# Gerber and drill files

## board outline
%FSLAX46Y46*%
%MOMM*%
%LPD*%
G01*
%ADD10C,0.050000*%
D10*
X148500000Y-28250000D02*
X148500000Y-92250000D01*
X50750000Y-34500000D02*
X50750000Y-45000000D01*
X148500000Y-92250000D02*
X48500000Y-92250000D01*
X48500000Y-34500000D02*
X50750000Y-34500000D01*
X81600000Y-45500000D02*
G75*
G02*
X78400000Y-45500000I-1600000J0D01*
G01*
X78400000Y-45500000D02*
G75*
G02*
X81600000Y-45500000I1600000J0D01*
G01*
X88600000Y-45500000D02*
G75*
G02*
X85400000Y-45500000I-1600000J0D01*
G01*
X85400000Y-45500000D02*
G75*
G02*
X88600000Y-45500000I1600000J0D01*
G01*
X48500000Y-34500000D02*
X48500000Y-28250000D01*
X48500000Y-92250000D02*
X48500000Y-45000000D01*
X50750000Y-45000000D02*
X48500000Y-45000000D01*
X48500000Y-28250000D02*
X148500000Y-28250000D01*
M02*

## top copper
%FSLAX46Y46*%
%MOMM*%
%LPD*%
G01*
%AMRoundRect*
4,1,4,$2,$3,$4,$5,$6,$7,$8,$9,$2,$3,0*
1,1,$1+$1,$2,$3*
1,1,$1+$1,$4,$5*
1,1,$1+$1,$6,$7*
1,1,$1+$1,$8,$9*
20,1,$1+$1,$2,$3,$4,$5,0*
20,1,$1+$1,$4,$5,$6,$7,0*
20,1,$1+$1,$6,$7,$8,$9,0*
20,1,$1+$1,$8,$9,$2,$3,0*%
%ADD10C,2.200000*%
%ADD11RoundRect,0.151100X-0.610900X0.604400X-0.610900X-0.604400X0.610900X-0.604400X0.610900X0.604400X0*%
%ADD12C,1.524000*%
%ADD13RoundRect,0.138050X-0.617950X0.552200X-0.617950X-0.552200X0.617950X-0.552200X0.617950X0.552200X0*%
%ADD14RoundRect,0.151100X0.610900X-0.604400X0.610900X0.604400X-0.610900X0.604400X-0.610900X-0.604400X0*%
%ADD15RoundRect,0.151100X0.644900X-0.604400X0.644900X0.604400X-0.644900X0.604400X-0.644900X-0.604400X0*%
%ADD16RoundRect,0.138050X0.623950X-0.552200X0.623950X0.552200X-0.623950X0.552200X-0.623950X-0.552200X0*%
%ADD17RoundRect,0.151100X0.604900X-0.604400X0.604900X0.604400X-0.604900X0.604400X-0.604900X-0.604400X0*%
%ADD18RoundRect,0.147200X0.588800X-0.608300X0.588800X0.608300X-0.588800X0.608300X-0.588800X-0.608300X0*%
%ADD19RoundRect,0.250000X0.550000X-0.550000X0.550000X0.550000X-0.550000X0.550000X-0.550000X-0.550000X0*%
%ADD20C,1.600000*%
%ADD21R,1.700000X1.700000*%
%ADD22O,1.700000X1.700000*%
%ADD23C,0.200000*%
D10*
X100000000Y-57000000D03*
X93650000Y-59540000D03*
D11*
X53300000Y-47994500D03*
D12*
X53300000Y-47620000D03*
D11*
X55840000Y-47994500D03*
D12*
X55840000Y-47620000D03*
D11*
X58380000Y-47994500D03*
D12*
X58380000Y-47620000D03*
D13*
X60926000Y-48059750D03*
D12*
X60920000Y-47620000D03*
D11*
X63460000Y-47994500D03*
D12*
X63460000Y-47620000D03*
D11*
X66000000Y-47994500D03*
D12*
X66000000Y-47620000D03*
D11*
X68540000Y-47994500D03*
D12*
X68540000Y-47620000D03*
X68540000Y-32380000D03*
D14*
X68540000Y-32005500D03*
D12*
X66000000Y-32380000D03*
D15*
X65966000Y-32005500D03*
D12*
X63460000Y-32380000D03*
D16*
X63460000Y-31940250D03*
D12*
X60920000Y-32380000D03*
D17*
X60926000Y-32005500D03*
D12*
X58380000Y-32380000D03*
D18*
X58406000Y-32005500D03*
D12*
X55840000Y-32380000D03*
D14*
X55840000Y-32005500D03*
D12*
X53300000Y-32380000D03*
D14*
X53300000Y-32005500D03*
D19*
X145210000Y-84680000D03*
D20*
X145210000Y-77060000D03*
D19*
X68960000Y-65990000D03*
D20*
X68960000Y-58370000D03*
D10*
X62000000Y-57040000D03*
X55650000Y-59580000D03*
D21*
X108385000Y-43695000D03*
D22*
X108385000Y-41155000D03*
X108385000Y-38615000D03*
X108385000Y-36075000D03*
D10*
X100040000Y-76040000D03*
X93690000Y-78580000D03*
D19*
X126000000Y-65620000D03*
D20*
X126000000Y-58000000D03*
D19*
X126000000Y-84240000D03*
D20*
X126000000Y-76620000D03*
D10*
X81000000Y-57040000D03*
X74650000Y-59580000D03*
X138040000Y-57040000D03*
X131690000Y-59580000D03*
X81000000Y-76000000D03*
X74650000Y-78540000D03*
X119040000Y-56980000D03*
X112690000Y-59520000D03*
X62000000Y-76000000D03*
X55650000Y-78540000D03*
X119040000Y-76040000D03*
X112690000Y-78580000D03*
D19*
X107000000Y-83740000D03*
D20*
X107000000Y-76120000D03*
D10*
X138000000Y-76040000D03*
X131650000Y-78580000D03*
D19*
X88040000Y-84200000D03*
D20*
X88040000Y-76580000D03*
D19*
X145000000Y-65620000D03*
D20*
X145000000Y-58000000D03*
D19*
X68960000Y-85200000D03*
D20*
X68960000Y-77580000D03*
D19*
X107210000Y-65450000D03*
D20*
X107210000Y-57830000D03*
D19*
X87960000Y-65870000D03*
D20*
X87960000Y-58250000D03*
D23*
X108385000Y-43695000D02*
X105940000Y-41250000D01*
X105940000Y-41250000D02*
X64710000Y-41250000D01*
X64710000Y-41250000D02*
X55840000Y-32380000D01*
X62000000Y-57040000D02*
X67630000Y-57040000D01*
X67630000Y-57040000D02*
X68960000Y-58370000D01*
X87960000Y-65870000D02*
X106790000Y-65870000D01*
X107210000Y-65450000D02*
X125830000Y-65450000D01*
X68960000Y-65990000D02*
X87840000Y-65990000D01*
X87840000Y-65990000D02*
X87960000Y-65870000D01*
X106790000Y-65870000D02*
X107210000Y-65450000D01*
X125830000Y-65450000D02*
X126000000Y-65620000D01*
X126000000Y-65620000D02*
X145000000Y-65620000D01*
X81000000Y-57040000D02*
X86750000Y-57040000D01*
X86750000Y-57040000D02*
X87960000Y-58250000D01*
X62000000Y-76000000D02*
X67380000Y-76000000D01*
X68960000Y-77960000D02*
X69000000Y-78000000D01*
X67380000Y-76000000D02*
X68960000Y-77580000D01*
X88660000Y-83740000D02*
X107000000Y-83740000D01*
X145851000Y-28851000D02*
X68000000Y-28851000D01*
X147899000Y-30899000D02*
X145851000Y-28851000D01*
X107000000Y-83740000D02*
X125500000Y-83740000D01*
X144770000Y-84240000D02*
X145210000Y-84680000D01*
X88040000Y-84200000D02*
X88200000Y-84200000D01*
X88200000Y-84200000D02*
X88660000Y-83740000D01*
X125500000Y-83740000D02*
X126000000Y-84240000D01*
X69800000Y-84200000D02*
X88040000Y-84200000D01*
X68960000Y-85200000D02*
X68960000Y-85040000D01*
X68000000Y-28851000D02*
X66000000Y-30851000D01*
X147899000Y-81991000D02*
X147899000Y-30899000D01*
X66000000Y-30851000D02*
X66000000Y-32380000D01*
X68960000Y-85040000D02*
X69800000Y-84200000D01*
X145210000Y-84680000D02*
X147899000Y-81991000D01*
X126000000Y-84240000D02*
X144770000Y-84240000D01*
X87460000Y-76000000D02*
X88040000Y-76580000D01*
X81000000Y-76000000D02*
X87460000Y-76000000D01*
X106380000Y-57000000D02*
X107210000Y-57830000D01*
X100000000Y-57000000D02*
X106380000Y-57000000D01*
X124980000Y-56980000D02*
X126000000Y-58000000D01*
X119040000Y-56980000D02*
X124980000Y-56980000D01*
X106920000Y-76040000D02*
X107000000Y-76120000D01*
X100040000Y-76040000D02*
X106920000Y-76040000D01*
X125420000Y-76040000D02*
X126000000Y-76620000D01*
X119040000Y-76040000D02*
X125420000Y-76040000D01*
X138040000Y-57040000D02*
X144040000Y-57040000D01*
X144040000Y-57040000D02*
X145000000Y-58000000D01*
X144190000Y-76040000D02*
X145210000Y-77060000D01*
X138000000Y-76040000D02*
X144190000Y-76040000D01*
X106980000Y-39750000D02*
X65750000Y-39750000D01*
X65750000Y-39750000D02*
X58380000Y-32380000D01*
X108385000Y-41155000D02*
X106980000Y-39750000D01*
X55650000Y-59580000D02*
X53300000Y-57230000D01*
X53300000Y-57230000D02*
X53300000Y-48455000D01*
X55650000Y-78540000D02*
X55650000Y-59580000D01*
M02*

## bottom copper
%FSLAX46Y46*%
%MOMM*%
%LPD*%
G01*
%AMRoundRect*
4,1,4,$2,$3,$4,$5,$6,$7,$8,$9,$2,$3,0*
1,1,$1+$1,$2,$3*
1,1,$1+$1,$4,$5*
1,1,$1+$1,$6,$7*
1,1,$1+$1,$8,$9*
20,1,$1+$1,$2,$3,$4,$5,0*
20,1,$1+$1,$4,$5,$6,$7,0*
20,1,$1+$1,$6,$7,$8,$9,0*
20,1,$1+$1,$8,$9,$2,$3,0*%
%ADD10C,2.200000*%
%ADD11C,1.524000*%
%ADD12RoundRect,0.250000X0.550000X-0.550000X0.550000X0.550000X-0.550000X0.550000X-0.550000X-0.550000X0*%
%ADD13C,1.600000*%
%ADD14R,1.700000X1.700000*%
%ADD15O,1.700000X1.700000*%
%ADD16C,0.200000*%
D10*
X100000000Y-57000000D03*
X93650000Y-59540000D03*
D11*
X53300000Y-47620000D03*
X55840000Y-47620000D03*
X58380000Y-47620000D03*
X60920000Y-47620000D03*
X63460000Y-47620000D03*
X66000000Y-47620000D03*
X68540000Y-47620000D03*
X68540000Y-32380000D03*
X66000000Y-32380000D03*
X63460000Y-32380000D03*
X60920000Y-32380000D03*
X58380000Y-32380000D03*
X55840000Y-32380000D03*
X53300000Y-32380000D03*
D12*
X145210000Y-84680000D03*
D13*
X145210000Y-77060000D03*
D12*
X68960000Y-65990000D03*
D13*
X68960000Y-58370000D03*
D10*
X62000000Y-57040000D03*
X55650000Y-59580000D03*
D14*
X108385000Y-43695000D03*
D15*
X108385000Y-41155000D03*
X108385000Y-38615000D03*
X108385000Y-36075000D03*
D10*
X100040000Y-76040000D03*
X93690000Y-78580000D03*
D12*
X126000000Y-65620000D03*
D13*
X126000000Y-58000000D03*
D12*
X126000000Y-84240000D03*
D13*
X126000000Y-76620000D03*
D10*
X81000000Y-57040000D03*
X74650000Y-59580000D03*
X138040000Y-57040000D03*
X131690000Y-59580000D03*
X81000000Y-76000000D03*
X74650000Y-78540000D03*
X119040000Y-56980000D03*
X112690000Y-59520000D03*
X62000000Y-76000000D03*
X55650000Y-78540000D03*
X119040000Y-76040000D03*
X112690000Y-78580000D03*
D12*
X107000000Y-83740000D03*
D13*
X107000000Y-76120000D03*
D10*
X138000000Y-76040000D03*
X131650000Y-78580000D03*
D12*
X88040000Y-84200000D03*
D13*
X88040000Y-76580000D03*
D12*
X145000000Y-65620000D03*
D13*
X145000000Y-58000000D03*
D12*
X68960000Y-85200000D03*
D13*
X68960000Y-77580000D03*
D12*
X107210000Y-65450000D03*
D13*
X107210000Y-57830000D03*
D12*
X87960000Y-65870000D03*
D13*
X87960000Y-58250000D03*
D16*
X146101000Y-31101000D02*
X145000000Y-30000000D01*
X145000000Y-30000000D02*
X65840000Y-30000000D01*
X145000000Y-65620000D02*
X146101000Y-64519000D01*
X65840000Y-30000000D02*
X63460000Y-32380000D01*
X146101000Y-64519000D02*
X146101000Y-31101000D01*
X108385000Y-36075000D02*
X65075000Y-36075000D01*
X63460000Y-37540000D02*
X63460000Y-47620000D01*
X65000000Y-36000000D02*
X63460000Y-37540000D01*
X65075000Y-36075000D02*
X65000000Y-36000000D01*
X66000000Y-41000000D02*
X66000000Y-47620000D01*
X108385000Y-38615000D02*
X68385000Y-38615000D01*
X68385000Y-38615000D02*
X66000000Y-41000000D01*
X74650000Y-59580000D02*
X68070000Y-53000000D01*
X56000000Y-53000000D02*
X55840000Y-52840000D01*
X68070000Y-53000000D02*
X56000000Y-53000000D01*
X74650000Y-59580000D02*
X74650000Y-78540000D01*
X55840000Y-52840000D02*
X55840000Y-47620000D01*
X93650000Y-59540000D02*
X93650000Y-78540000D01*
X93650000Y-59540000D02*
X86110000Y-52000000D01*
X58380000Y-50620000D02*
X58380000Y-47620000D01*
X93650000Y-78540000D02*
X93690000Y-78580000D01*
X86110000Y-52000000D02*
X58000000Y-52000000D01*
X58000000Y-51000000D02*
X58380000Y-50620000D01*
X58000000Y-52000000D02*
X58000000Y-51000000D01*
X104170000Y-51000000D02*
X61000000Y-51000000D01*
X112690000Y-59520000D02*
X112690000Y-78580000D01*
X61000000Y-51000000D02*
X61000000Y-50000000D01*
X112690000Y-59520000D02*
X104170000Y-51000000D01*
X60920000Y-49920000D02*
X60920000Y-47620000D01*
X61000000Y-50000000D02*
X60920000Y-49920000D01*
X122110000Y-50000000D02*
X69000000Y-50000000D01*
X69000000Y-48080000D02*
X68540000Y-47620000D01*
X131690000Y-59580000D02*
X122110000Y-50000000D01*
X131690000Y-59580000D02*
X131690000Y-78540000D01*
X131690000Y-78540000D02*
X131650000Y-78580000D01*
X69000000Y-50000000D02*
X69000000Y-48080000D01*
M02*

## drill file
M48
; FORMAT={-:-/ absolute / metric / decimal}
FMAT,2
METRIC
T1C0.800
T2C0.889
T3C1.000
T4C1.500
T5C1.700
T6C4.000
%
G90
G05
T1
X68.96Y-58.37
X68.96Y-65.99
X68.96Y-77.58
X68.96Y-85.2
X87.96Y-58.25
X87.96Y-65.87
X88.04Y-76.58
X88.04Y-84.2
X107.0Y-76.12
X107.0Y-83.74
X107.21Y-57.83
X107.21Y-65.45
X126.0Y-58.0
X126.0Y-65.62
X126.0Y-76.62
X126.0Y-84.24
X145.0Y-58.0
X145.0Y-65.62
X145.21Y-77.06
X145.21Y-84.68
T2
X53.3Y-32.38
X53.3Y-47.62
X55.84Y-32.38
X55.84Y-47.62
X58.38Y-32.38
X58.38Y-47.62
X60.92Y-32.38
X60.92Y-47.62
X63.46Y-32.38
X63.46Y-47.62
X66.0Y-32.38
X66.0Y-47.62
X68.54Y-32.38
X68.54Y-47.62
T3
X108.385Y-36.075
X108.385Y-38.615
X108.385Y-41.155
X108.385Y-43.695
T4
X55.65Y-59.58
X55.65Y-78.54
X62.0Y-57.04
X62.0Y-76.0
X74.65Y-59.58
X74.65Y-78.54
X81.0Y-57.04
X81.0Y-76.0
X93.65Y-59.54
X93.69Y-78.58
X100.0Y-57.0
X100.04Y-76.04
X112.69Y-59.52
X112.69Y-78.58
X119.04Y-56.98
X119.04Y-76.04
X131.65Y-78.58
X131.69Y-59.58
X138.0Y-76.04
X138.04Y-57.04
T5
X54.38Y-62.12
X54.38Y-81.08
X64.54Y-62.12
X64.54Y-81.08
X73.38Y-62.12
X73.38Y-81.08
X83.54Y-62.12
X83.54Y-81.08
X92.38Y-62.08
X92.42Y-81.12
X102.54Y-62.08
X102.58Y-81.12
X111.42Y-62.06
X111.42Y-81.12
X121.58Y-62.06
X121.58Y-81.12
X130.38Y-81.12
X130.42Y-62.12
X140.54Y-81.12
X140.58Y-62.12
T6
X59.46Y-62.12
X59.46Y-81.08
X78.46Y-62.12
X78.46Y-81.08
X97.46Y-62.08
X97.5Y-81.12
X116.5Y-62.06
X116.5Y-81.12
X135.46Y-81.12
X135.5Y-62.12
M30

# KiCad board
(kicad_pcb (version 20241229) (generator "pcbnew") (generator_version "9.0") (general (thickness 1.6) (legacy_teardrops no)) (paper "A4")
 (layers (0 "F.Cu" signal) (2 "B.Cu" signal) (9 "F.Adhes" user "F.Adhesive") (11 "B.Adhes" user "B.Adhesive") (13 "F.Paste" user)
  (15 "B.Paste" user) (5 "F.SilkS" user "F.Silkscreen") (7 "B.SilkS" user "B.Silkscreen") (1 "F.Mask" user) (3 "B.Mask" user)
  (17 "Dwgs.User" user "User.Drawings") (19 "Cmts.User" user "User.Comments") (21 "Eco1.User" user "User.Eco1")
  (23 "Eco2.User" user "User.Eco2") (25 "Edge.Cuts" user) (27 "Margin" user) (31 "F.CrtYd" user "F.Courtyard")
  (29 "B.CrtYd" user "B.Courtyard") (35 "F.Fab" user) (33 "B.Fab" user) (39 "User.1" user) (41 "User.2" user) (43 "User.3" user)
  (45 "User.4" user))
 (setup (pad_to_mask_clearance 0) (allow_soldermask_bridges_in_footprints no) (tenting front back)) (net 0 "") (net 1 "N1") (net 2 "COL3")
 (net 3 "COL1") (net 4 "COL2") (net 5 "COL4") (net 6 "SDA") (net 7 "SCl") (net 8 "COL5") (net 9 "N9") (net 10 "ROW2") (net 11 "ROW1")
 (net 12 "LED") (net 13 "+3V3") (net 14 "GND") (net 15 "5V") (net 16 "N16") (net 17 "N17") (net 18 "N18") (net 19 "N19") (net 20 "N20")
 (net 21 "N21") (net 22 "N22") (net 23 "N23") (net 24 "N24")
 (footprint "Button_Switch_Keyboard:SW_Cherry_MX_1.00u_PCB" (layer "F.Cu") (at 100 57)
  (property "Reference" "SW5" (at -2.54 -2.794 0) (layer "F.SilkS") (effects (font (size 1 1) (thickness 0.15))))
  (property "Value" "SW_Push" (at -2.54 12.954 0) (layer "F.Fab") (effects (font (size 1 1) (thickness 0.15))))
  (pad "" np_thru_hole circle (at -7.62 5.08) (size 1.7 1.7) (drill 1.7) (layers "*.Cu" "*.Mask"))
  (pad "" np_thru_hole circle (at -2.54 5.08) (size 4 4) (drill 4) (layers "*.Cu" "*.Mask"))
  (pad "" np_thru_hole circle (at 2.54 5.08) (size 1.7 1.7) (drill 1.7) (layers "*.Cu" "*.Mask"))
  (pad "1" thru_hole circle (at 0 0) (size 2.2 2.2) (drill 1.5) (layers "*.Cu" "*.Mask") (remove_unused_layers no) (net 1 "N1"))
  (pad "2" thru_hole circle (at -6.35 2.54) (size 2.2 2.2) (drill 1.5) (layers "*.Cu" "*.Mask") (remove_unused_layers no) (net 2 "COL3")))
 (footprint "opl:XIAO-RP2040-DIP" (layer "F.Cu") (at 60.92 40 90)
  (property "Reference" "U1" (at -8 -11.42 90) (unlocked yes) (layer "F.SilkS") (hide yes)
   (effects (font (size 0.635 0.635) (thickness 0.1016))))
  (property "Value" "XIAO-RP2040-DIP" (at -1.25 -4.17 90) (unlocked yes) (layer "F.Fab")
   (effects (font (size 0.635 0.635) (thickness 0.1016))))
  (pad "1" smd roundrect (at -7.9945 -7.62 270) (size 1.511 1.524) (layers "F.Cu" "F.Mask") (roundrect_rratio 0.1) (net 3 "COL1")
   (thermal_bridge_angle 45))
  (pad "1" thru_hole circle (at -7.62 -7.62 270) (size 1.524 1.524) (drill 0.889) (layers "*.Cu" "*.Mask") (remove_unused_layers no)
   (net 3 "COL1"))
  (pad "2" smd roundrect (at -7.9945 -5.08 270) (size 1.511 1.524) (layers "F.Cu" "F.Mask") (roundrect_rratio 0.1) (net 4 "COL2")
   (thermal_bridge_angle 45))
  (pad "2" thru_hole circle (at -7.62 -5.08 270) (size 1.524 1.524) (drill 0.889) (layers "*.Cu" "*.Mask") (remove_unused_layers no)
   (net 4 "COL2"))
  (pad "3" smd roundrect (at -7.9945 -2.54 270) (size 1.511 1.524) (layers "F.Cu" "F.Mask") (roundrect_rratio 0.1) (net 2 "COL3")
   (thermal_bridge_angle 45))
  (pad "3" thru_hole circle (at -7.62 -2.54 270) (size 1.524 1.524) (drill 0.889) (layers "*.Cu" "*.Mask") (remove_unused_layers no)
   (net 2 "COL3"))
  (pad "4" smd roundrect (at -8.05975 0.006 270) (size 1.3805 1.512) (layers "F.Cu" "F.Mask") (roundrect_rratio 0.1) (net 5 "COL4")
   (thermal_bridge_angle 45))
  (pad "4" thru_hole circle (at -7.62 0 270) (size 1.524 1.524) (drill 0.889) (layers "*.Cu" "*.Mask") (remove_unused_layers no)
   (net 5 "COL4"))
  (pad "5" smd roundrect (at -7.9945 2.54 270) (size 1.511 1.524) (layers "F.Cu" "F.Mask") (roundrect_rratio 0.1) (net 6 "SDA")
   (thermal_bridge_angle 45))
  (pad "5" thru_hole circle (at -7.62 2.54 270) (size 1.524 1.524) (drill 0.889) (layers "*.Cu" "*.Mask") (remove_unused_layers no)
   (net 6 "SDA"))
  (pad "6" smd roundrect (at -7.9945 5.08 270) (size 1.511 1.524) (layers "F.Cu" "F.Mask") (roundrect_rratio 0.1) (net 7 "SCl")
   (thermal_bridge_angle 45))
  (pad "6" thru_hole circle (at -7.62 5.08 270) (size 1.524 1.524) (drill 0.889) (layers "*.Cu" "*.Mask") (remove_unused_layers no)
   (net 7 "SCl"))
  (pad "7" smd roundrect (at -7.9945 7.62 270) (size 1.511 1.524) (layers "F.Cu" "F.Mask") (roundrect_rratio 0.1) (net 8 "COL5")
   (thermal_bridge_angle 45))
  (pad "7" thru_hole circle (at -7.62 7.62 270) (size 1.524 1.524) (drill 0.889) (layers "*.Cu" "*.Mask") (remove_unused_layers no)
   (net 8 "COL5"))
  (pad "8" thru_hole circle (at 7.62 7.62 90) (size 1.524 1.524) (drill 0.889) (layers "*.Cu" "*.Mask") (remove_unused_layers no)
   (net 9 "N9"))
  (pad "8" smd roundrect (at 7.9945 7.62 90) (size 1.511 1.524) (layers "F.Cu" "F.Mask") (roundrect_rratio 0.1) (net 9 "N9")
   (thermal_bridge_angle 45))
  (pad "9" thru_hole circle (at 7.62 5.08 90) (size 1.524 1.524) (drill 0.889) (layers "*.Cu" "*.Mask") (remove_unused_layers no)
   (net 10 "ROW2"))
  (pad "9" smd roundrect (at 7.9945 5.046 90) (size 1.511 1.592) (layers "F.Cu" "F.Mask") (roundrect_rratio 0.1) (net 10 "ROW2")
   (thermal_bridge_angle 45))
  (pad "10" thru_hole circle (at 7.62 2.54 90) (size 1.524 1.524) (drill 0.889) (layers "*.Cu" "*.Mask") (remove_unused_layers no)
   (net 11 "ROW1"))
  (pad "10" smd roundrect (at 8.05975 2.54 90) (size 1.3805 1.524) (layers "F.Cu" "F.Mask") (roundrect_rratio 0.1) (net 11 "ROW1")
   (thermal_bridge_angle 45))
  (pad "11" thru_hole circle (at 7.62 0 90) (size 1.524 1.524) (drill 0.889) (layers "*.Cu" "*.Mask") (remove_unused_layers no)
   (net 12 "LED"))
  (pad "11" smd roundrect (at 7.9945 0.006 90) (size 1.511 1.512) (layers "F.Cu" "F.Mask") (roundrect_rratio 0.1) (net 12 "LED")
   (thermal_bridge_angle 45))
  (pad "12" thru_hole circle (at 7.62 -2.54 90) (size 1.524 1.524) (drill 0.889) (layers "*.Cu" "*.Mask") (remove_unused_layers no)
   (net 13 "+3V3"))
  (pad "12" smd roundrect (at 7.9945 -2.514 90) (size 1.511 1.472) (layers "F.Cu" "F.Mask") (roundrect_rratio 0.1) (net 13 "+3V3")
   (thermal_bridge_angle 45))
  (pad "13" thru_hole circle (at 7.62 -5.08 90) (size 1.524 1.524) (drill 0.889) (layers "*.Cu" "*.Mask") (remove_unused_layers no)
   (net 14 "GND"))
  (pad "13" smd roundrect (at 7.9945 -5.08 90) (size 1.511 1.524) (layers "F.Cu" "F.Mask") (roundrect_rratio 0.1) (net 14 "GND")
   (thermal_bridge_angle 45))
  (pad "14" thru_hole circle (at 7.62 -7.62 90) (size 1.524 1.524) (drill 0.889) (layers "*.Cu" "*.Mask") (remove_unused_layers no)
   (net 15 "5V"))
  (pad "14" smd roundrect (at 7.9945 -7.62 90) (size 1.511 1.524) (layers "F.Cu" "F.Mask") (roundrect_rratio 0.1) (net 15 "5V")
   (thermal_bridge_angle 45)))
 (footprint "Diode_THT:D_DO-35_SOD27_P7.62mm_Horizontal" (layer "F.Cu") (at 145.21 84.68 90)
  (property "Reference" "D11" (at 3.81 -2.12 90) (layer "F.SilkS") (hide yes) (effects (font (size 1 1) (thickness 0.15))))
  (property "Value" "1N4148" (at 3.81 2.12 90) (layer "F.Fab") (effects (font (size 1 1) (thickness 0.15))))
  (pad "1" thru_hole roundrect (at 0 0 90) (size 1.6 1.6) (drill 0.8) (layers "*.Cu" "*.Mask") (remove_unused_layers no)
   (roundrect_rratio 0.15625) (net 10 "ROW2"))
  (pad "2" thru_hole circle (at 7.62 0 90) (size 1.6 1.6) (drill 0.8) (layers "*.Cu" "*.Mask") (remove_unused_layers no) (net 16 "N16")))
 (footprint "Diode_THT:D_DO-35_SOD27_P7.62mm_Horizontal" (layer "F.Cu") (at 68.96 65.99 90)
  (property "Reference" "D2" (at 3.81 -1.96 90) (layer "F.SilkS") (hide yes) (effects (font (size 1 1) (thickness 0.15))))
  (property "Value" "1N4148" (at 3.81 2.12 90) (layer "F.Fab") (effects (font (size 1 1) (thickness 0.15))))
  (pad "1" thru_hole roundrect (at 0 0 90) (size 1.6 1.6) (drill 0.8) (layers "*.Cu" "*.Mask") (remove_unused_layers no)
   (roundrect_rratio 0.15625) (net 11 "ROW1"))
  (pad "2" thru_hole circle (at 7.62 0 90) (size 1.6 1.6) (drill 0.8) (layers "*.Cu" "*.Mask") (remove_unused_layers no) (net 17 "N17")))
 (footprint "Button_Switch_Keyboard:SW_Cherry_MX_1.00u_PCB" (layer "F.Cu") (at 62 57.04)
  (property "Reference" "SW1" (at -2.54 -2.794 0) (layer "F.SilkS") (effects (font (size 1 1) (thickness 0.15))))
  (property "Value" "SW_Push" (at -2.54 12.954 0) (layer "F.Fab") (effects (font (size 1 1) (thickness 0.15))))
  (pad "" np_thru_hole circle (at -7.62 5.08) (size 1.7 1.7) (drill 1.7) (layers "*.Cu" "*.Mask"))
  (pad "" np_thru_hole circle (at -2.54 5.08) (size 4 4) (drill 4) (layers "*.Cu" "*.Mask"))
  (pad "" np_thru_hole circle (at 2.54 5.08) (size 1.7 1.7) (drill 1.7) (layers "*.Cu" "*.Mask"))
  (pad "1" thru_hole circle (at 0 0) (size 2.2 2.2) (drill 1.5) (layers "*.Cu" "*.Mask") (remove_unused_layers no) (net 17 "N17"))
  (pad "2" thru_hole circle (at -6.35 2.54) (size 2.2 2.2) (drill 1.5) (layers "*.Cu" "*.Mask") (remove_unused_layers no) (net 3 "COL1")))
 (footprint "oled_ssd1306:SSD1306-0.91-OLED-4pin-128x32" (layer "F.Cu") (at 144.885 45.885 180)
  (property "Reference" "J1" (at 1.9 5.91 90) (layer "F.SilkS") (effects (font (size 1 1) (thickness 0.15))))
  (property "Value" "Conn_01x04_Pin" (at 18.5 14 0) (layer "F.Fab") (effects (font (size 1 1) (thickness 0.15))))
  (pad "1" thru_hole rect (at 36.5 2.19 180) (size 1.7 1.7) (drill 1) (layers "*.Cu" "*.Mask") (remove_unused_layers no) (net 14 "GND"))
  (pad "2" thru_hole oval (at 36.5 4.73 180) (size 1.7 1.7) (drill 1) (layers "*.Cu" "*.Mask") (remove_unused_layers no) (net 13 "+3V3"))
  (pad "3" thru_hole oval (at 36.5 7.27 180) (size 1.7 1.7) (drill 1) (layers "*.Cu" "*.Mask") (remove_unused_layers no) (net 7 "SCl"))
  (pad "4" thru_hole oval (at 36.5 9.81 180) (size 1.7 1.7) (drill 1) (layers "*.Cu" "*.Mask") (remove_unused_layers no) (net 6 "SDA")))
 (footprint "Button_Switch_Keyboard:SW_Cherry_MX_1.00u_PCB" (layer "F.Cu") (at 100.04 76.04)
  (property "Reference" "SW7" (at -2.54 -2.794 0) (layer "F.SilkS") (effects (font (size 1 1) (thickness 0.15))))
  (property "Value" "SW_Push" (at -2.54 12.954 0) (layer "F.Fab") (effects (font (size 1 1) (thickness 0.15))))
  (pad "" np_thru_hole circle (at -7.62 5.08) (size 1.7 1.7) (drill 1.7) (layers "*.Cu" "*.Mask"))
  (pad "" np_thru_hole circle (at -2.54 5.08) (size 4 4) (drill 4) (layers "*.Cu" "*.Mask"))
  (pad "" np_thru_hole circle (at 2.54 5.08) (size 1.7 1.7) (drill 1.7) (layers "*.Cu" "*.Mask"))
  (pad "1" thru_hole circle (at 0 0) (size 2.2 2.2) (drill 1.5) (layers "*.Cu" "*.Mask") (remove_unused_layers no) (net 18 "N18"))
  (pad "2" thru_hole circle (at -6.35 2.54) (size 2.2 2.2) (drill 1.5) (layers "*.Cu" "*.Mask") (remove_unused_layers no) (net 2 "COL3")))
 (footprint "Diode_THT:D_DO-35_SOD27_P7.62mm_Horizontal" (layer "F.Cu") (at 126 65.62 90)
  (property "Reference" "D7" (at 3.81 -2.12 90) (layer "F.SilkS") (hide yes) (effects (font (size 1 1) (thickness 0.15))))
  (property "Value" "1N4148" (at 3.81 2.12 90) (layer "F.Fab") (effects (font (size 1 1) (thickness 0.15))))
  (pad "1" thru_hole roundrect (at 0 0 90) (size 1.6 1.6) (drill 0.8) (layers "*.Cu" "*.Mask") (remove_unused_layers no)
   (roundrect_rratio 0.15625) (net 11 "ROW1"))
  (pad "2" thru_hole circle (at 7.62 0 90) (size 1.6 1.6) (drill 0.8) (layers "*.Cu" "*.Mask") (remove_unused_layers no) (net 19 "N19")))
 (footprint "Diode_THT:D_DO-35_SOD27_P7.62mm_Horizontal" (layer "F.Cu") (at 126 84.24 90)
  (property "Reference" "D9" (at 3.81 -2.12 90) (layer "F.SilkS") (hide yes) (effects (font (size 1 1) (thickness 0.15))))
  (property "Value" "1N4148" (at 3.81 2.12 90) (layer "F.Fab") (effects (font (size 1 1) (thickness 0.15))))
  (pad "1" thru_hole roundrect (at 0 0 90) (size 1.6 1.6) (drill 0.8) (layers "*.Cu" "*.Mask") (remove_unused_layers no)
   (roundrect_rratio 0.15625) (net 10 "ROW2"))
  (pad "2" thru_hole circle (at 7.62 0 90) (size 1.6 1.6) (drill 0.8) (layers "*.Cu" "*.Mask") (remove_unused_layers no) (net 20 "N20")))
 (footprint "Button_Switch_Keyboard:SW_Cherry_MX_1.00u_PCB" (layer "F.Cu") (at 81 57.04)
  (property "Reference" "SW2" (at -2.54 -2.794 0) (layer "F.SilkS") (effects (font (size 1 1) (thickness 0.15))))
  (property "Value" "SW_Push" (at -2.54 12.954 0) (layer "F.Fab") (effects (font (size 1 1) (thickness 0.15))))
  (pad "" np_thru_hole circle (at -7.62 5.08) (size 1.7 1.7) (drill 1.7) (layers "*.Cu" "*.Mask"))
  (pad "" np_thru_hole circle (at -2.54 5.08) (size 4 4) (drill 4) (layers "*.Cu" "*.Mask"))
  (pad "" np_thru_hole circle (at 2.54 5.08) (size 1.7 1.7) (drill 1.7) (layers "*.Cu" "*.Mask"))
  (pad "1" thru_hole circle (at 0 0) (size 2.2 2.2) (drill 1.5) (layers "*.Cu" "*.Mask") (remove_unused_layers no) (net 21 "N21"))
  (pad "2" thru_hole circle (at -6.35 2.54) (size 2.2 2.2) (drill 1.5) (layers "*.Cu" "*.Mask") (remove_unused_layers no) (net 4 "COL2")))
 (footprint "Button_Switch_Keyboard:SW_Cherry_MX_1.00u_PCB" (layer "F.Cu") (at 138.04 57.04)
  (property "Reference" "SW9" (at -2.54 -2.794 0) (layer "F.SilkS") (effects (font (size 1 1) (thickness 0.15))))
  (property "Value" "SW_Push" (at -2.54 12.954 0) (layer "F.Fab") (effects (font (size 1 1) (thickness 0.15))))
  (pad "" np_thru_hole circle (at -7.62 5.08) (size 1.7 1.7) (drill 1.7) (layers "*.Cu" "*.Mask"))
  (pad "" np_thru_hole circle (at -2.54 5.08) (size 4 4) (drill 4) (layers "*.Cu" "*.Mask"))
  (pad "" np_thru_hole circle (at 2.54 5.08) (size 1.7 1.7) (drill 1.7) (layers "*.Cu" "*.Mask"))
  (pad "1" thru_hole circle (at 0 0) (size 2.2 2.2) (drill 1.5) (layers "*.Cu" "*.Mask") (remove_unused_layers no) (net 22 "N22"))
  (pad "2" thru_hole circle (at -6.35 2.54) (size 2.2 2.2) (drill 1.5) (layers "*.Cu" "*.Mask") (remove_unused_layers no) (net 8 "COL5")))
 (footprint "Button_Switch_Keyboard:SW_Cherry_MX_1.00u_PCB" (layer "F.Cu") (at 81 76)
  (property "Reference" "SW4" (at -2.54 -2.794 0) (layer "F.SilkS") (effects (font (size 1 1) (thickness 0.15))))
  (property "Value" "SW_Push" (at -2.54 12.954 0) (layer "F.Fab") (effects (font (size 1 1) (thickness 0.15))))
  (pad "" np_thru_hole circle (at -7.62 5.08) (size 1.7 1.7) (drill 1.7) (layers "*.Cu" "*.Mask"))
  (pad "" np_thru_hole circle (at -2.54 5.08) (size 4 4) (drill 4) (layers "*.Cu" "*.Mask"))
  (pad "" np_thru_hole circle (at 2.54 5.08) (size 1.7 1.7) (drill 1.7) (layers "*.Cu" "*.Mask"))
  (pad "1" thru_hole circle (at 0 0) (size 2.2 2.2) (drill 1.5) (layers "*.Cu" "*.Mask") (remove_unused_layers no) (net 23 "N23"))
  (pad "2" thru_hole circle (at -6.35 2.54) (size 2.2 2.2) (drill 1.5) (layers "*.Cu" "*.Mask") (remove_unused_layers no) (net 4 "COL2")))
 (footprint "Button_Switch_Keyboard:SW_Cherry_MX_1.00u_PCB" (layer "F.Cu") (at 119.04 56.98)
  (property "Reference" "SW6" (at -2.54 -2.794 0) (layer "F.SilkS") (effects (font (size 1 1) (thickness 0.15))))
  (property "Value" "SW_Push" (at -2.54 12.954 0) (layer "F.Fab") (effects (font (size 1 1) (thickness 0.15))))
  (pad "" np_thru_hole circle (at -7.62 5.08) (size 1.7 1.7) (drill 1.7) (layers "*.Cu" "*.Mask"))
  (pad "" np_thru_hole circle (at -2.54 5.08) (size 4 4) (drill 4) (layers "*.Cu" "*.Mask"))
  (pad "" np_thru_hole circle (at 2.54 5.08) (size 1.7 1.7) (drill 1.7) (layers "*.Cu" "*.Mask"))
  (pad "1" thru_hole circle (at 0 0) (size 2.2 2.2) (drill 1.5) (layers "*.Cu" "*.Mask") (remove_unused_layers no) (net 19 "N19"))
  (pad "2" thru_hole circle (at -6.35 2.54) (size 2.2 2.2) (drill 1.5) (layers "*.Cu" "*.Mask") (remove_unused_layers no) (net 5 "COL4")))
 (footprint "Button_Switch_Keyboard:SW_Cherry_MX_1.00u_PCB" (layer "F.Cu") (at 62 76)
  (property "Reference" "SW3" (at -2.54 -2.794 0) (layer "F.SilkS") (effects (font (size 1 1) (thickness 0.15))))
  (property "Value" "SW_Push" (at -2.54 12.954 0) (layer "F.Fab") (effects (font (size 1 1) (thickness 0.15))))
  (pad "" np_thru_hole circle (at -7.62 5.08) (size 1.7 1.7) (drill 1.7) (layers "*.Cu" "*.Mask"))
  (pad "" np_thru_hole circle (at -2.54 5.08) (size 4 4) (drill 4) (layers "*.Cu" "*.Mask"))
  (pad "" np_thru_hole circle (at 2.54 5.08) (size 1.7 1.7) (drill 1.7) (layers "*.Cu" "*.Mask"))
  (pad "1" thru_hole circle (at 0 0) (size 2.2 2.2) (drill 1.5) (layers "*.Cu" "*.Mask") (remove_unused_layers no) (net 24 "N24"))
  (pad "2" thru_hole circle (at -6.35 2.54) (size 2.2 2.2) (drill 1.5) (layers "*.Cu" "*.Mask") (remove_unused_layers no) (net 3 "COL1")))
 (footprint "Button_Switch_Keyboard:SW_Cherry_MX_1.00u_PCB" (layer "F.Cu") (at 119.04 76.04)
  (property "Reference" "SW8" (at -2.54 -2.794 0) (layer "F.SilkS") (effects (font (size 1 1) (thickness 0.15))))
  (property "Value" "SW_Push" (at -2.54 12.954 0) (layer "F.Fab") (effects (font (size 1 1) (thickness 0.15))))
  (pad "" np_thru_hole circle (at -7.62 5.08) (size 1.7 1.7) (drill 1.7) (layers "*.Cu" "*.Mask"))
  (pad "" np_thru_hole circle (at -2.54 5.08) (size 4 4) (drill 4) (layers "*.Cu" "*.Mask"))
  (pad "" np_thru_hole circle (at 2.54 5.08) (size 1.7 1.7) (drill 1.7) (layers "*.Cu" "*.Mask"))
  (pad "1" thru_hole circle (at 0 0) (size 2.2 2.2) (drill 1.5) (layers "*.Cu" "*.Mask") (remove_unused_layers no) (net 20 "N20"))
  (pad "2" thru_hole circle (at -6.35 2.54) (size 2.2 2.2) (drill 1.5) (layers "*.Cu" "*.Mask") (remove_unused_layers no) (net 5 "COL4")))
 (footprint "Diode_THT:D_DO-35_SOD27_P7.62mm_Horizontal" (layer "F.Cu") (at 107 83.74 90)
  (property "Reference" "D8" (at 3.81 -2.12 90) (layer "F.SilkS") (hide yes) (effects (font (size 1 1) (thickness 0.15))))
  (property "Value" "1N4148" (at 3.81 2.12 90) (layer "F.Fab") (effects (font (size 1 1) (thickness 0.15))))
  (pad "1" thru_hole roundrect (at 0 0 90) (size 1.6 1.6) (drill 0.8) (layers "*.Cu" "*.Mask") (remove_unused_layers no)
   (roundrect_rratio 0.15625) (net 10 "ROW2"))
  (pad "2" thru_hole circle (at 7.62 0 90) (size 1.6 1.6) (drill 0.8) (layers "*.Cu" "*.Mask") (remove_unused_layers no) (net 18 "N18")))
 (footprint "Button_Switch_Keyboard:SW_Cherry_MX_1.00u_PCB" (layer "F.Cu") (at 138 76.04)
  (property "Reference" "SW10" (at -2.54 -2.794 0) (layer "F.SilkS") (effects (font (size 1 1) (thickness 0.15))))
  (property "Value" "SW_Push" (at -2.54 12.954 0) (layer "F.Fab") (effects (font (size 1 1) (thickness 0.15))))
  (pad "" np_thru_hole circle (at -7.62 5.08) (size 1.7 1.7) (drill 1.7) (layers "*.Cu" "*.Mask"))
  (pad "" np_thru_hole circle (at -2.54 5.08) (size 4 4) (drill 4) (layers "*.Cu" "*.Mask"))
  (pad "" np_thru_hole circle (at 2.54 5.08) (size 1.7 1.7) (drill 1.7) (layers "*.Cu" "*.Mask"))
  (pad "1" thru_hole circle (at 0 0) (size 2.2 2.2) (drill 1.5) (layers "*.Cu" "*.Mask") (remove_unused_layers no) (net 16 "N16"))
  (pad "2" thru_hole circle (at -6.35 2.54) (size 2.2 2.2) (drill 1.5) (layers "*.Cu" "*.Mask") (remove_unused_layers no) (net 8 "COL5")))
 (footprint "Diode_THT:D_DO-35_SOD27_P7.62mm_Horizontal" (layer "F.Cu") (at 88.04 84.2 90)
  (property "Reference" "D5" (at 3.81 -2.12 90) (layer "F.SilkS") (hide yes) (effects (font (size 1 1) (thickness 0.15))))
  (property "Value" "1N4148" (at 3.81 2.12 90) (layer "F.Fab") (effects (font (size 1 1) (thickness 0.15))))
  (pad "1" thru_hole roundrect (at 0 0 90) (size 1.6 1.6) (drill 0.8) (layers "*.Cu" "*.Mask") (remove_unused_layers no)
   (roundrect_rratio 0.15625) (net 10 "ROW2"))
  (pad "2" thru_hole circle (at 7.62 0 90) (size 1.6 1.6) (drill 0.8) (layers "*.Cu" "*.Mask") (remove_unused_layers no) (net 23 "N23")))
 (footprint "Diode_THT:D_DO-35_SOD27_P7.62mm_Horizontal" (layer "F.Cu") (at 145 65.62 90)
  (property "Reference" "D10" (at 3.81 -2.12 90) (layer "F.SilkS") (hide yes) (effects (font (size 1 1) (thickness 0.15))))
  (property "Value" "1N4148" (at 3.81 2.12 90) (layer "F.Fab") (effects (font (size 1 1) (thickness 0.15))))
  (pad "1" thru_hole roundrect (at 0 0 90) (size 1.6 1.6) (drill 0.8) (layers "*.Cu" "*.Mask") (remove_unused_layers no)
   (roundrect_rratio 0.15625) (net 11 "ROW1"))
  (pad "2" thru_hole circle (at 7.62 0 90) (size 1.6 1.6) (drill 0.8) (layers "*.Cu" "*.Mask") (remove_unused_layers no) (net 22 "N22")))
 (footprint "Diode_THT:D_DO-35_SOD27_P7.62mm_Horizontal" (layer "F.Cu") (at 68.96 85.2 90)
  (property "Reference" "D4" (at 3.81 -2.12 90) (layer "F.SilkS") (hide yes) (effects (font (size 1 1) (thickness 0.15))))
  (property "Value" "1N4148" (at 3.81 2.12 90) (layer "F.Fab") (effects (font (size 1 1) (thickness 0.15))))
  (pad "1" thru_hole roundrect (at 0 0 90) (size 1.6 1.6) (drill 0.8) (layers "*.Cu" "*.Mask") (remove_unused_layers no)
   (roundrect_rratio 0.15625) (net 10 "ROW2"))
  (pad "2" thru_hole circle (at 7.62 0 90) (size 1.6 1.6) (drill 0.8) (layers "*.Cu" "*.Mask") (remove_unused_layers no) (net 24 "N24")))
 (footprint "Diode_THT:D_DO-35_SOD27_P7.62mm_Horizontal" (layer "F.Cu") (at 107.21 65.45 90)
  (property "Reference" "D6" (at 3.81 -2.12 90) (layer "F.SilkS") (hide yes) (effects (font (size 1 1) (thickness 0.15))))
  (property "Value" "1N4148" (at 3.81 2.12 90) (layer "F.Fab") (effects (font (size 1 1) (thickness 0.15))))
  (pad "1" thru_hole roundrect (at 0 0 90) (size 1.6 1.6) (drill 0.8) (layers "*.Cu" "*.Mask") (remove_unused_layers no)
   (roundrect_rratio 0.15625) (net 11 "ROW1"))
  (pad "2" thru_hole circle (at 7.62 0 90) (size 1.6 1.6) (drill 0.8) (layers "*.Cu" "*.Mask") (remove_unused_layers no) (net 1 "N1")))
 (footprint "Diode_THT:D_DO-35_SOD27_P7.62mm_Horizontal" (layer "F.Cu") (at 87.96 65.87 90)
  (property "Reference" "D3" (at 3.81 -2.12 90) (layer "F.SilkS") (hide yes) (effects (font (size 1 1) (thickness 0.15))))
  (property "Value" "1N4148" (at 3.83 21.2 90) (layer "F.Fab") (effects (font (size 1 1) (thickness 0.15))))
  (pad "1" thru_hole roundrect (at 0 0 90) (size 1.6 1.6) (drill 0.8) (layers "*.Cu" "*.Mask") (remove_unused_layers no)
   (roundrect_rratio 0.15625) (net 11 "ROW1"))
  (pad "2" thru_hole circle (at 7.62 0 90) (size 1.6 1.6) (drill 0.8) (layers "*.Cu" "*.Mask") (remove_unused_layers no) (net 21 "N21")))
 (gr_line (start 148.5 28.25) (end 148.5 92.25) (stroke (width 0.05) (type default)) (layer "Edge.Cuts"))
 (gr_line (start 50.75 34.5) (end 50.75 45) (stroke (width 0.05) (type default)) (layer "Edge.Cuts"))
 (gr_line (start 148.5 92.25) (end 48.5 92.25) (stroke (width 0.05) (type default)) (layer "Edge.Cuts"))
 (gr_line (start 48.5 34.5) (end 50.75 34.5) (stroke (width 0.05) (type default)) (layer "Edge.Cuts"))
 (gr_circle (center 80 45.5) (end 81.6 45.5) (stroke (width 0.05) (type solid)) (fill no) (layer "Edge.Cuts"))
 (gr_circle (center 87 45.5) (end 88.6 45.5) (stroke (width 0.05) (type solid)) (fill no) (layer "Edge.Cuts"))
 (gr_line (start 48.5 34.5) (end 48.5 28.25) (stroke (width 0.05) (type default)) (layer "Edge.Cuts"))
 (gr_line (start 48.5 92.25) (end 48.5 45) (stroke (width 0.05) (type default)) (layer "Edge.Cuts"))
 (gr_line (start 50.75 45) (end 48.5 45) (stroke (width 0.05) (type default)) (layer "Edge.Cuts"))
 (gr_line (start 48.5 28.25) (end 148.5 28.25) (stroke (width 0.05) (type default)) (layer "Edge.Cuts"))
 (segment (start 108.385 43.695) (end 105.94 41.25) (width 0.2) (layer "F.Cu") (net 14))
 (segment (start 105.94 41.25) (end 64.71 41.25) (width 0.2) (layer "F.Cu") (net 14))
 (segment (start 64.71 41.25) (end 55.84 32.38) (width 0.2) (layer "F.Cu") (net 14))
 (segment (start 62 57.04) (end 67.63 57.04) (width 0.2) (layer "F.Cu") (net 17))
 (segment (start 67.63 57.04) (end 68.96 58.37) (width 0.2) (layer "F.Cu") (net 17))
 (segment (start 87.96 65.87) (end 106.79 65.87) (width 0.2) (layer "F.Cu") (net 11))
 (segment (start 107.21 65.45) (end 125.83 65.45) (width 0.2) (layer "F.Cu") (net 11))
 (segment (start 68.96 65.99) (end 87.84 65.99) (width 0.2) (layer "F.Cu") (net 11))
 (segment (start 87.84 65.99) (end 87.96 65.87) (width 0.2) (layer "F.Cu") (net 11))
 (segment (start 106.79 65.87) (end 107.21 65.45) (width 0.2) (layer "F.Cu") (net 11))
 (segment (start 125.83 65.45) (end 126 65.62) (width 0.2) (layer "F.Cu") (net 11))
 (segment (start 126 65.62) (end 145 65.62) (width 0.2) (layer "F.Cu") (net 11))
 (segment (start 146.101 31.101) (end 145 30) (width 0.2) (layer "B.Cu") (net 11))
 (segment (start 145 30) (end 65.84 30) (width 0.2) (layer "B.Cu") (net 11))
 (segment (start 145 65.62) (end 146.101 64.519) (width 0.2) (layer "B.Cu") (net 11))
 (segment (start 65.84 30) (end 63.46 32.38) (width 0.2) (layer "B.Cu") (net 11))
 (segment (start 146.101 64.519) (end 146.101 31.101) (width 0.2) (layer "B.Cu") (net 11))
 (segment (start 81 57.04) (end 86.75 57.04) (width 0.2) (layer "F.Cu") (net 21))
 (segment (start 86.75 57.04) (end 87.96 58.25) (width 0.2) (layer "F.Cu") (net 21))
 (segment (start 62 76) (end 67.38 76) (width 0.2) (layer "F.Cu") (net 24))
 (segment (start 68.96 77.96) (end 69 78) (width 0.2) (layer "F.Cu") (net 24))
 (segment (start 67.38 76) (end 68.96 77.58) (width 0.2) (layer "F.Cu") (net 24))
 (segment (start 88.66 83.74) (end 107 83.74) (width 0.2) (layer "F.Cu") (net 10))
 (segment (start 145.851 28.851) (end 68 28.851) (width 0.2) (layer "F.Cu") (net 10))
 (segment (start 147.899 30.899) (end 145.851 28.851) (width 0.2) (layer "F.Cu") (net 10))
 (segment (start 107 83.74) (end 125.5 83.74) (width 0.2) (layer "F.Cu") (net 10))
 (segment (start 144.77 84.24) (end 145.21 84.68) (width 0.2) (layer "F.Cu") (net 10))
 (segment (start 88.04 84.2) (end 88.2 84.2) (width 0.2) (layer "F.Cu") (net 10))
 (segment (start 88.2 84.2) (end 88.66 83.74) (width 0.2) (layer "F.Cu") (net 10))
 (segment (start 125.5 83.74) (end 126 84.24) (width 0.2) (layer "F.Cu") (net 10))
 (segment (start 69.8 84.2) (end 88.04 84.2) (width 0.2) (layer "F.Cu") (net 10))
 (segment (start 68.96 85.2) (end 68.96 85.04) (width 0.2) (layer "F.Cu") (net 10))
 (segment (start 68 28.851) (end 66 30.851) (width 0.2) (layer "F.Cu") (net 10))
 (segment (start 147.899 81.991) (end 147.899 30.899) (width 0.2) (layer "F.Cu") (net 10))
 (segment (start 66 30.851) (end 66 32.38) (width 0.2) (layer "F.Cu") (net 10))
 (segment (start 68.96 85.04) (end 69.8 84.2) (width 0.2) (layer "F.Cu") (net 10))
 (segment (start 145.21 84.68) (end 147.899 81.991) (width 0.2) (layer "F.Cu") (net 10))
 (segment (start 126 84.24) (end 144.77 84.24) (width 0.2) (layer "F.Cu") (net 10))
 (segment (start 87.46 76) (end 88.04 76.58) (width 0.2) (layer "F.Cu") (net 23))
 (segment (start 81 76) (end 87.46 76) (width 0.2) (layer "F.Cu") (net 23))
 (segment (start 106.38 57) (end 107.21 57.83) (width 0.2) (layer "F.Cu") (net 1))
 (segment (start 100 57) (end 106.38 57) (width 0.2) (layer "F.Cu") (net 1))
 (segment (start 124.98 56.98) (end 126 58) (width 0.2) (layer "F.Cu") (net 19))
 (segment (start 119.04 56.98) (end 124.98 56.98) (width 0.2) (layer "F.Cu") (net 19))
 (segment (start 106.92 76.04) (end 107 76.12) (width 0.2) (layer "F.Cu") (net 18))
 (segment (start 100.04 76.04) (end 106.92 76.04) (width 0.2) (layer "F.Cu") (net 18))
 (segment (start 125.42 76.04) (end 126 76.62) (width 0.2) (layer "F.Cu") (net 20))
 (segment (start 119.04 76.04) (end 125.42 76.04) (width 0.2) (layer "F.Cu") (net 20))
 (segment (start 138.04 57.04) (end 144.04 57.04) (width 0.2) (layer "F.Cu") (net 22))
 (segment (start 144.04 57.04) (end 145 58) (width 0.2) (layer "F.Cu") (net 22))
 (segment (start 144.19 76.04) (end 145.21 77.06) (width 0.2) (layer "F.Cu") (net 16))
 (segment (start 138 76.04) (end 144.19 76.04) (width 0.2) (layer "F.Cu") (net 16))
 (segment (start 106.98 39.75) (end 65.75 39.75) (width 0.2) (layer "F.Cu") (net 13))
 (segment (start 65.75 39.75) (end 58.38 32.38) (width 0.2) (layer "F.Cu") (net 13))
 (segment (start 108.385 41.155) (end 106.98 39.75) (width 0.2) (layer "F.Cu") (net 13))
 (segment (start 108.385 36.075) (end 65.075 36.075) (width 0.2) (layer "B.Cu") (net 6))
 (segment (start 63.46 37.54) (end 63.46 47.62) (width 0.2) (layer "B.Cu") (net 6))
 (segment (start 65 36) (end 63.46 37.54) (width 0.2) (layer "B.Cu") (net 6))
 (segment (start 65.075 36.075) (end 65 36) (width 0.2) (layer "B.Cu") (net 6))
 (segment (start 66 41) (end 66 47.62) (width 0.2) (layer "B.Cu") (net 7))
 (segment (start 108.385 38.615) (end 68.385 38.615) (width 0.2) (layer "B.Cu") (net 7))
 (segment (start 68.385 38.615) (end 66 41) (width 0.2) (layer "B.Cu") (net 7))
 (segment (start 55.65 59.58) (end 53.3 57.23) (width 0.2) (layer "F.Cu") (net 3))
 (segment (start 53.3 57.23) (end 53.3 48.455) (width 0.2) (layer "F.Cu") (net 3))
 (segment (start 55.65 78.54) (end 55.65 59.58) (width 0.2) (layer "F.Cu") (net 3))
 (segment (start 74.65 59.58) (end 68.07 53) (width 0.2) (layer "B.Cu") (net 4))
 (segment (start 56 53) (end 55.84 52.84) (width 0.2) (layer "B.Cu") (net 4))
 (segment (start 68.07 53) (end 56 53) (width 0.2) (layer "B.Cu") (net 4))
 (segment (start 74.65 59.58) (end 74.65 78.54) (width 0.2) (layer "B.Cu") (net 4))
 (segment (start 55.84 52.84) (end 55.84 47.62) (width 0.2) (layer "B.Cu") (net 4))
 (segment (start 93.65 59.54) (end 93.65 78.54) (width 0.2) (layer "B.Cu") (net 2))
 (segment (start 93.65 59.54) (end 86.11 52) (width 0.2) (layer "B.Cu") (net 2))
 (segment (start 58.38 50.62) (end 58.38 47.62) (width 0.2) (layer "B.Cu") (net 2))
 (segment (start 93.65 78.54) (end 93.69 78.58) (width 0.2) (layer "B.Cu") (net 2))
 (segment (start 86.11 52) (end 58 52) (width 0.2) (layer "B.Cu") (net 2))
 (segment (start 58 51) (end 58.38 50.62) (width 0.2) (layer "B.Cu") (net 2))
 (segment (start 58 52) (end 58 51) (width 0.2) (layer "B.Cu") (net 2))
 (segment (start 104.17 51) (end 61 51) (width 0.2) (layer "B.Cu") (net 5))
 (segment (start 112.69 59.52) (end 112.69 78.58) (width 0.2) (layer "B.Cu") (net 5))
 (segment (start 61 51) (end 61 50) (width 0.2) (layer "B.Cu") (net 5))
 (segment (start 112.69 59.52) (end 104.17 51) (width 0.2) (layer "B.Cu") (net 5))
 (segment (start 60.92 49.92) (end 60.92 47.62) (width 0.2) (layer "B.Cu") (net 5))
 (segment (start 61 50) (end 60.92 49.92) (width 0.2) (layer "B.Cu") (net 5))
 (segment (start 122.11 50) (end 69 50) (width 0.2) (layer "B.Cu") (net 8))
 (segment (start 69 48.08) (end 68.54 47.62) (width 0.2) (layer "B.Cu") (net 8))
 (segment (start 131.69 59.58) (end 122.11 50) (width 0.2) (layer "B.Cu") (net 8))
 (segment (start 131.69 59.58) (end 131.69 78.54) (width 0.2) (layer "B.Cu") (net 8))
 (segment (start 131.69 78.54) (end 131.65 78.58) (width 0.2) (layer "B.Cu") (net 8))
 (segment (start 69 50) (end 69 48.08) (width 0.2) (layer "B.Cu") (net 8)))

